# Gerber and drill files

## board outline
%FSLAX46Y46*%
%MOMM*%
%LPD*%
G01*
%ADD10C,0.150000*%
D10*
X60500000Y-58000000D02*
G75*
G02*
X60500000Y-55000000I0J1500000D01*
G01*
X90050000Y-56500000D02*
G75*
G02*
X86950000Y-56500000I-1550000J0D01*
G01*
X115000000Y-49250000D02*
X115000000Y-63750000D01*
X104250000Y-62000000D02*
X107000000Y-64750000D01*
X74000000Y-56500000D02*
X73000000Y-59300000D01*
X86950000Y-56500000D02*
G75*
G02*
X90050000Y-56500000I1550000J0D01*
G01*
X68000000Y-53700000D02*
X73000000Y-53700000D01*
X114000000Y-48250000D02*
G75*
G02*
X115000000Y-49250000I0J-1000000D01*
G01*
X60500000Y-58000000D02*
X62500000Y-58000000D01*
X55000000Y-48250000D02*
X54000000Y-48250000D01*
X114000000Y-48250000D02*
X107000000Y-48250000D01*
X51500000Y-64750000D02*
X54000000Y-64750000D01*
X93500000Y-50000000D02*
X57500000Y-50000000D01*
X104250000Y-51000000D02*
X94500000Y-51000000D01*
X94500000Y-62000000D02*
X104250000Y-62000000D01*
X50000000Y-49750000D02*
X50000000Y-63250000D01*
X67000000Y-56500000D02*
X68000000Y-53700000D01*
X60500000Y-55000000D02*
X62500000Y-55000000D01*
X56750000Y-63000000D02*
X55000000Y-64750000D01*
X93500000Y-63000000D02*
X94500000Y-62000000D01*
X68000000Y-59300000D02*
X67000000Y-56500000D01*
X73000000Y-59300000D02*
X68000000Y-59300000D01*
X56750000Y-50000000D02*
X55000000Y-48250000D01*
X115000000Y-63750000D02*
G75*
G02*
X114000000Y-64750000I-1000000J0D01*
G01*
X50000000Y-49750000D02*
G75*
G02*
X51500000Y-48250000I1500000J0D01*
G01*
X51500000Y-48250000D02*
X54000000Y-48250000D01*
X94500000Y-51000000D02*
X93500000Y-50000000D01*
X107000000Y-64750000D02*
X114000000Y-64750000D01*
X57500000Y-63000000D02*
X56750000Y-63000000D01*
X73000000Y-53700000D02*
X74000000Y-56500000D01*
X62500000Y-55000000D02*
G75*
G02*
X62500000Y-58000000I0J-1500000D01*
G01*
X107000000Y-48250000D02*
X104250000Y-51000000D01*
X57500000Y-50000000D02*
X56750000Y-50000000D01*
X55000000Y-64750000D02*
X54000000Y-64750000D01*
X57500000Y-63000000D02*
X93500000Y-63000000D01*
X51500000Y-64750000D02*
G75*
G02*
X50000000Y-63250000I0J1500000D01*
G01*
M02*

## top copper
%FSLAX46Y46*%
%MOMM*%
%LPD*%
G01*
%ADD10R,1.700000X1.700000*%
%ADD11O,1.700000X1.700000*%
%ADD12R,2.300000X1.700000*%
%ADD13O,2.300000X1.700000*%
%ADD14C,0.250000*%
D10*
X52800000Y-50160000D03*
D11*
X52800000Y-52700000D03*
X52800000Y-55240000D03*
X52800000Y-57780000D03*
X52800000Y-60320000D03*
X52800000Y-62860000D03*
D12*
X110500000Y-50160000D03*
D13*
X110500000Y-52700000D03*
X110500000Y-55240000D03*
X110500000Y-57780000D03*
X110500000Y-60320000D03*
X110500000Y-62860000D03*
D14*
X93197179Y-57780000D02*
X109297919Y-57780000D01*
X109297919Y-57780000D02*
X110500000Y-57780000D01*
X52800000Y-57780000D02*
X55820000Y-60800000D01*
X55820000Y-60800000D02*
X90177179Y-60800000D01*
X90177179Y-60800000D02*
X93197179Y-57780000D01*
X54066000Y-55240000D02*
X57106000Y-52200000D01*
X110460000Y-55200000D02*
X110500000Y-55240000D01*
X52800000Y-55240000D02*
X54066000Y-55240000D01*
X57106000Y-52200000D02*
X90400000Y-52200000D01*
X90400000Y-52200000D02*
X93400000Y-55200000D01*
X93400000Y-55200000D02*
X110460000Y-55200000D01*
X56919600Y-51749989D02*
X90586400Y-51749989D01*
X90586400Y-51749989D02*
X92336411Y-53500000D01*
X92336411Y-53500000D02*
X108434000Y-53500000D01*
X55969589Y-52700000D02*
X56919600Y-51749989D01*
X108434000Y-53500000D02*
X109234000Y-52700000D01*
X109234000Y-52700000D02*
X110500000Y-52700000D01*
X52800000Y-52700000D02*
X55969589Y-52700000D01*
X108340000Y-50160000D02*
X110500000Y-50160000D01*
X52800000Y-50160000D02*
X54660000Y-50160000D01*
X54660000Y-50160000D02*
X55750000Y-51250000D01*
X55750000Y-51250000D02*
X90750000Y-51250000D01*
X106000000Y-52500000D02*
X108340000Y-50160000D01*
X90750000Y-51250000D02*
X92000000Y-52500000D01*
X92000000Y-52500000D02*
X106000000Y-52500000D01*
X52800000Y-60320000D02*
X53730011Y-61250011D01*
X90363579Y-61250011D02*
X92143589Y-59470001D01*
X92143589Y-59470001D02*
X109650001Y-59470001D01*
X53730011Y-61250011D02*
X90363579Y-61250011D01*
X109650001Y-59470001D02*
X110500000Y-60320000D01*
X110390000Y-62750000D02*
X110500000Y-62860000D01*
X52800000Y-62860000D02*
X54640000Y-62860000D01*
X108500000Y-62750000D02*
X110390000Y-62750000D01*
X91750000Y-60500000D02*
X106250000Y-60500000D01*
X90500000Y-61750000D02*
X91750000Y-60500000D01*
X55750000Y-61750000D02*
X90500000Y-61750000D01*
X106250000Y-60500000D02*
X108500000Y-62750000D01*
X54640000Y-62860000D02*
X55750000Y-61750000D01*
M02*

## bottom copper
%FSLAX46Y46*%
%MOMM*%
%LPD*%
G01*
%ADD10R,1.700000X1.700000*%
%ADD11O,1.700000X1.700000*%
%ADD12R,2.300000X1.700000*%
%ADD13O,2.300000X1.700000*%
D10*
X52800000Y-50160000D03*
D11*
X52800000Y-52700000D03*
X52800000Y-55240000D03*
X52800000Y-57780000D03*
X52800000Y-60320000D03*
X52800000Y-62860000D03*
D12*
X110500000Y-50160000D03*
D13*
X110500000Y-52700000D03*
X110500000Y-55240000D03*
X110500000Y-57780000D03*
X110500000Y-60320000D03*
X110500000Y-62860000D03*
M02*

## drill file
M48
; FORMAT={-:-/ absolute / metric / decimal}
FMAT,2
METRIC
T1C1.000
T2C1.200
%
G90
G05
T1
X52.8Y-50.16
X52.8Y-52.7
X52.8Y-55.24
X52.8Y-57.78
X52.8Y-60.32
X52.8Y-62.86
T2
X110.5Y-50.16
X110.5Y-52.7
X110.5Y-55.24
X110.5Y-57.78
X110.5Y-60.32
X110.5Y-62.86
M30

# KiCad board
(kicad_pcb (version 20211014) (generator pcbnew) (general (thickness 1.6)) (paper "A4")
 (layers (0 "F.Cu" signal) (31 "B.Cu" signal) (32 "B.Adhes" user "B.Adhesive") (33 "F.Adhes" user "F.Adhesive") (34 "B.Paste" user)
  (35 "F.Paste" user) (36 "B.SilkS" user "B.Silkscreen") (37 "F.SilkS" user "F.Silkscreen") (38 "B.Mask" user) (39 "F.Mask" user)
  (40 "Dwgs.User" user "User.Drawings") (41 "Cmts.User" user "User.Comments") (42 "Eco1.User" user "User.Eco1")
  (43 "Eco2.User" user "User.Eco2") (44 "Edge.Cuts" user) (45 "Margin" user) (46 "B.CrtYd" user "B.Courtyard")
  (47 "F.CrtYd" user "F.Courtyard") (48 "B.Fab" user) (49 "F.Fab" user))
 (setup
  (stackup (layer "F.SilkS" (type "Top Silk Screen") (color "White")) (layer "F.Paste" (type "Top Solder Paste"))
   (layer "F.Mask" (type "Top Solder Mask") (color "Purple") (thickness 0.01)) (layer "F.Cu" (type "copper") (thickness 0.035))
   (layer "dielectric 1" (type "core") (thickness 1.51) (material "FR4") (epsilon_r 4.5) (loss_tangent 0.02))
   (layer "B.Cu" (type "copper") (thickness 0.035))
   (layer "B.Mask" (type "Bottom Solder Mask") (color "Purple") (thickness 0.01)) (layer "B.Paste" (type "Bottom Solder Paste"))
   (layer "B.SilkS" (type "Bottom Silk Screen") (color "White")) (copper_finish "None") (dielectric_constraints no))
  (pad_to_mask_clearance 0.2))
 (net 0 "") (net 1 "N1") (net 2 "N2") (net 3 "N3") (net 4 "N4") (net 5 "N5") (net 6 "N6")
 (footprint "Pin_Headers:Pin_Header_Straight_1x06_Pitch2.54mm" (layer "F.Cu") (at 52.8 50.16)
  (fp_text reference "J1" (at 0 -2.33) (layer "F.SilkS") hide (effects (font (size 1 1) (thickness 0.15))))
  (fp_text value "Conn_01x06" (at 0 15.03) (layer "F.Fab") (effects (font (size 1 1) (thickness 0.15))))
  (pad "1" thru_hole rect locked (at 0 0) (size 1.7 1.7) (drill 1) (layers *.Cu *.Mask) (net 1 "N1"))
  (pad "2" thru_hole oval locked (at 0 2.54) (size 1.7 1.7) (drill 1) (layers *.Cu *.Mask) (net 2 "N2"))
  (pad "3" thru_hole oval locked (at 0 5.08) (size 1.7 1.7) (drill 1) (layers *.Cu *.Mask) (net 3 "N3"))
  (pad "4" thru_hole oval locked (at 0 7.62) (size 1.7 1.7) (drill 1) (layers *.Cu *.Mask) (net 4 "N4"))
  (pad "5" thru_hole oval locked (at 0 10.16) (size 1.7 1.7) (drill 1) (layers *.Cu *.Mask) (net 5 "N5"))
  (pad "6" thru_hole oval locked (at 0 12.7) (size 1.7 1.7) (drill 1) (layers *.Cu *.Mask) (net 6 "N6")))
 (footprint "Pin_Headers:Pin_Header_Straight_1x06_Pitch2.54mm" (layer "F.Cu") (at 110.5 50.16)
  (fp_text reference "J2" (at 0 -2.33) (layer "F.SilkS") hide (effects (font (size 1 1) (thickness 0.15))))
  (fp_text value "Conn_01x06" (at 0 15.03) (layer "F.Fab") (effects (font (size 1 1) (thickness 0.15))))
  (pad "1" thru_hole rect locked (at 0 0) (size 2.3 1.7) (drill 1.2) (layers *.Cu *.Mask) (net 1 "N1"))
  (pad "2" thru_hole oval locked (at 0 2.54) (size 2.3 1.7) (drill 1.2) (layers *.Cu *.Mask) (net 2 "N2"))
  (pad "3" thru_hole oval locked (at 0 5.08) (size 2.3 1.7) (drill 1.2) (layers *.Cu *.Mask) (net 3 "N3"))
  (pad "4" thru_hole oval locked (at 0 7.62) (size 2.3 1.7) (drill 1.2) (layers *.Cu *.Mask) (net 4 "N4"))
  (pad "5" thru_hole oval locked (at 0 10.16) (size 2.3 1.7) (drill 1.2) (layers *.Cu *.Mask) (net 5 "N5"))
  (pad "6" thru_hole oval locked (at 0 12.7) (size 2.3 1.7) (drill 1.2) (layers *.Cu *.Mask) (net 6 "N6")))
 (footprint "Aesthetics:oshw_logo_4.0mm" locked (layer "F.Cu") (at 99.695 56.515 -90)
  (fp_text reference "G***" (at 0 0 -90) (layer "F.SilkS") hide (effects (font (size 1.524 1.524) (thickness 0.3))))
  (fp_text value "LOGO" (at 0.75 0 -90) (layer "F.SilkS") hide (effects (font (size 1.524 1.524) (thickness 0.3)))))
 (gr_arc (start 60.5 58) (mid 59 56.5) (end 60.5 55) (layer "Edge.Cuts") (width 0.15))
 (gr_arc (start 90.05 56.5) (mid 88.5 58.05) (end 86.95 56.5) (layer "Edge.Cuts") (width 0.15))
 (gr_line (start 115 49.25) (end 115 63.75) (layer "Edge.Cuts") (width 0.15))
 (gr_line (start 104.25 62) (end 107 64.75) (layer "Edge.Cuts") (width 0.15))
 (gr_line (start 74 56.5) (end 73 59.3) (layer "Edge.Cuts") (width 0.15))
 (gr_arc (start 86.95 56.5) (mid 88.5 54.95) (end 90.05 56.5) (layer "Edge.Cuts") (width 0.15))
 (gr_line (start 68 53.7) (end 73 53.7) (layer "Edge.Cuts") (width 0.15))
 (gr_arc (start 114 48.25) (mid 114.707107 48.542893) (end 115 49.25) (layer "Edge.Cuts") (width 0.15))
 (gr_line (start 60.5 58) (end 62.5 58) (layer "Edge.Cuts") (width 0.15))
 (gr_line (start 55 48.25) (end 54 48.25) (layer "Edge.Cuts") (width 0.15))
 (gr_line (start 114 48.25) (end 107 48.25) (layer "Edge.Cuts") (width 0.15))
 (gr_line (start 51.5 64.75) (end 54 64.75) (layer "Edge.Cuts") (width 0.15))
 (gr_line (start 93.5 50) (end 57.5 50) (layer "Edge.Cuts") (width 0.15))
 (gr_line (start 104.25 51) (end 94.5 51) (layer "Edge.Cuts") (width 0.15))
 (gr_line (start 94.5 62) (end 104.25 62) (layer "Edge.Cuts") (width 0.15))
 (gr_line (start 50 49.75) (end 50 63.25) (layer "Edge.Cuts") (width 0.15))
 (gr_line (start 67 56.5) (end 68 53.7) (layer "Edge.Cuts") (width 0.15))
 (gr_line (start 60.5 55) (end 62.5 55) (layer "Edge.Cuts") (width 0.15))
 (gr_line (start 56.75 63) (end 55 64.75) (layer "Edge.Cuts") (width 0.15))
 (gr_line (start 93.5 63) (end 94.5 62) (layer "Edge.Cuts") (width 0.15))
 (gr_line (start 68 59.3) (end 67 56.5) (layer "Edge.Cuts") (width 0.15))
 (gr_line (start 73 59.3) (end 68 59.3) (layer "Edge.Cuts") (width 0.15))
 (gr_line (start 56.75 50) (end 55 48.25) (layer "Edge.Cuts") (width 0.15))
 (gr_arc (start 115 63.75) (mid 114.707107 64.457107) (end 114 64.75) (layer "Edge.Cuts") (width 0.15))
 (gr_arc (start 50 49.75) (mid 50.43934 48.68934) (end 51.5 48.25) (layer "Edge.Cuts") (width 0.15))
 (gr_line (start 51.5 48.25) (end 54 48.25) (layer "Edge.Cuts") (width 0.15))
 (gr_line (start 94.5 51) (end 93.5 50) (layer "Edge.Cuts") (width 0.15))
 (gr_line (start 107 64.75) (end 114 64.75) (layer "Edge.Cuts") (width 0.15))
 (gr_line (start 57.5 63) (end 56.75 63) (layer "Edge.Cuts") (width 0.15))
 (gr_line (start 73 53.7) (end 74 56.5) (layer "Edge.Cuts") (width 0.15))
 (gr_arc (start 62.5 55) (mid 64 56.5) (end 62.5 58) (layer "Edge.Cuts") (width 0.15))
 (gr_line (start 107 48.25) (end 104.25 51) (layer "Edge.Cuts") (width 0.15))
 (gr_line (start 57.5 50) (end 56.75 50) (layer "Edge.Cuts") (width 0.15))
 (gr_line (start 55 64.75) (end 54 64.75) (layer "Edge.Cuts") (width 0.15))
 (gr_line (start 57.5 63) (end 93.5 63) (layer "Edge.Cuts") (width 0.15))
 (gr_arc (start 51.5 64.75) (mid 50.43934 64.31066) (end 50 63.25) (layer "Edge.Cuts") (width 0.15))
 (segment (start 93.197179 57.78) (end 109.297919 57.78) (width 0.25) (layer "F.Cu") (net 4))
 (segment (start 109.297919 57.78) (end 110.5 57.78) (width 0.25) (layer "F.Cu") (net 4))
 (segment (start 52.8 57.78) (end 55.82 60.8) (width 0.25) (layer "F.Cu") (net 4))
 (segment (start 55.82 60.8) (end 90.177179 60.8) (width 0.25) (layer "F.Cu") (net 4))
 (segment (start 90.177179 60.8) (end 93.197179 57.78) (width 0.25) (layer "F.Cu") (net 4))
 (segment (start 54.066 55.24) (end 57.106 52.2) (width 0.25) (layer "F.Cu") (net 3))
 (segment (start 110.46 55.2) (end 110.5 55.24) (width 0.25) (layer "F.Cu") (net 3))
 (segment (start 52.8 55.24) (end 54.066 55.24) (width 0.25) (layer "F.Cu") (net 3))
 (segment (start 57.106 52.2) (end 90.4 52.2) (width 0.25) (layer "F.Cu") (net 3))
 (segment (start 90.4 52.2) (end 93.4 55.2) (width 0.25) (layer "F.Cu") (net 3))
 (segment (start 93.4 55.2) (end 110.46 55.2) (width 0.25) (layer "F.Cu") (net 3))
 (segment (start 56.9196 51.749989) (end 90.5864 51.749989) (width 0.25) (layer "F.Cu") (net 2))
 (segment (start 90.5864 51.749989) (end 92.336411 53.5) (width 0.25) (layer "F.Cu") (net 2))
 (segment (start 92.336411 53.5) (end 108.434 53.5) (width 0.25) (layer "F.Cu") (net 2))
 (segment (start 55.969589 52.7) (end 56.9196 51.749989) (width 0.25) (layer "F.Cu") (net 2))
 (segment (start 108.434 53.5) (end 109.234 52.7) (width 0.25) (layer "F.Cu") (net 2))
 (segment (start 109.234 52.7) (end 110.5 52.7) (width 0.25) (layer "F.Cu") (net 2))
 (segment (start 52.8 52.7) (end 55.969589 52.7) (width 0.25) (layer "F.Cu") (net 2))
 (segment (start 108.34 50.16) (end 110.5 50.16) (width 0.25) (layer "F.Cu") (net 1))
 (segment (start 52.8 50.16) (end 54.66 50.16) (width 0.25) (layer "F.Cu") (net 1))
 (segment (start 54.66 50.16) (end 55.75 51.25) (width 0.25) (layer "F.Cu") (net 1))
 (segment (start 55.75 51.25) (end 90.75 51.25) (width 0.25) (layer "F.Cu") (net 1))
 (segment (start 106 52.5) (end 108.34 50.16) (width 0.25) (layer "F.Cu") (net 1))
 (segment (start 90.75 51.25) (end 92 52.5) (width 0.25) (layer "F.Cu") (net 1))
 (segment (start 92 52.5) (end 106 52.5) (width 0.25) (layer "F.Cu") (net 1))
 (segment (start 52.8 60.32) (end 53.730011 61.250011) (width 0.25) (layer "F.Cu") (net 5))
 (segment (start 90.363579 61.250011) (end 92.143589 59.470001) (width 0.25) (layer "F.Cu") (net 5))
 (segment (start 92.143589 59.470001) (end 109.650001 59.470001) (width 0.25) (layer "F.Cu") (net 5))
 (segment (start 53.730011 61.250011) (end 90.363579 61.250011) (width 0.25) (layer "F.Cu") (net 5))
 (segment (start 109.650001 59.470001) (end 110.5 60.32) (width 0.25) (layer "F.Cu") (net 5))
 (segment (start 110.39 62.75) (end 110.5 62.86) (width 0.25) (layer "F.Cu") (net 6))
 (segment (start 52.8 62.86) (end 54.64 62.86) (width 0.25) (layer "F.Cu") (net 6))
 (segment (start 108.5 62.75) (end 110.39 62.75) (width 0.25) (layer "F.Cu") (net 6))
 (segment (start 91.75 60.5) (end 106.25 60.5) (width 0.25) (layer "F.Cu") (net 6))
 (segment (start 90.5 61.75) (end 91.75 60.5) (width 0.25) (layer "F.Cu") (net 6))
 (segment (start 55.75 61.75) (end 90.5 61.75) (width 0.25) (layer "F.Cu") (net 6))
 (segment (start 106.25 60.5) (end 108.5 62.75) (width 0.25) (layer "F.Cu") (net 6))
 (segment (start 54.64 62.86) (end 55.75 61.75) (width 0.25) (layer "F.Cu") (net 6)))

